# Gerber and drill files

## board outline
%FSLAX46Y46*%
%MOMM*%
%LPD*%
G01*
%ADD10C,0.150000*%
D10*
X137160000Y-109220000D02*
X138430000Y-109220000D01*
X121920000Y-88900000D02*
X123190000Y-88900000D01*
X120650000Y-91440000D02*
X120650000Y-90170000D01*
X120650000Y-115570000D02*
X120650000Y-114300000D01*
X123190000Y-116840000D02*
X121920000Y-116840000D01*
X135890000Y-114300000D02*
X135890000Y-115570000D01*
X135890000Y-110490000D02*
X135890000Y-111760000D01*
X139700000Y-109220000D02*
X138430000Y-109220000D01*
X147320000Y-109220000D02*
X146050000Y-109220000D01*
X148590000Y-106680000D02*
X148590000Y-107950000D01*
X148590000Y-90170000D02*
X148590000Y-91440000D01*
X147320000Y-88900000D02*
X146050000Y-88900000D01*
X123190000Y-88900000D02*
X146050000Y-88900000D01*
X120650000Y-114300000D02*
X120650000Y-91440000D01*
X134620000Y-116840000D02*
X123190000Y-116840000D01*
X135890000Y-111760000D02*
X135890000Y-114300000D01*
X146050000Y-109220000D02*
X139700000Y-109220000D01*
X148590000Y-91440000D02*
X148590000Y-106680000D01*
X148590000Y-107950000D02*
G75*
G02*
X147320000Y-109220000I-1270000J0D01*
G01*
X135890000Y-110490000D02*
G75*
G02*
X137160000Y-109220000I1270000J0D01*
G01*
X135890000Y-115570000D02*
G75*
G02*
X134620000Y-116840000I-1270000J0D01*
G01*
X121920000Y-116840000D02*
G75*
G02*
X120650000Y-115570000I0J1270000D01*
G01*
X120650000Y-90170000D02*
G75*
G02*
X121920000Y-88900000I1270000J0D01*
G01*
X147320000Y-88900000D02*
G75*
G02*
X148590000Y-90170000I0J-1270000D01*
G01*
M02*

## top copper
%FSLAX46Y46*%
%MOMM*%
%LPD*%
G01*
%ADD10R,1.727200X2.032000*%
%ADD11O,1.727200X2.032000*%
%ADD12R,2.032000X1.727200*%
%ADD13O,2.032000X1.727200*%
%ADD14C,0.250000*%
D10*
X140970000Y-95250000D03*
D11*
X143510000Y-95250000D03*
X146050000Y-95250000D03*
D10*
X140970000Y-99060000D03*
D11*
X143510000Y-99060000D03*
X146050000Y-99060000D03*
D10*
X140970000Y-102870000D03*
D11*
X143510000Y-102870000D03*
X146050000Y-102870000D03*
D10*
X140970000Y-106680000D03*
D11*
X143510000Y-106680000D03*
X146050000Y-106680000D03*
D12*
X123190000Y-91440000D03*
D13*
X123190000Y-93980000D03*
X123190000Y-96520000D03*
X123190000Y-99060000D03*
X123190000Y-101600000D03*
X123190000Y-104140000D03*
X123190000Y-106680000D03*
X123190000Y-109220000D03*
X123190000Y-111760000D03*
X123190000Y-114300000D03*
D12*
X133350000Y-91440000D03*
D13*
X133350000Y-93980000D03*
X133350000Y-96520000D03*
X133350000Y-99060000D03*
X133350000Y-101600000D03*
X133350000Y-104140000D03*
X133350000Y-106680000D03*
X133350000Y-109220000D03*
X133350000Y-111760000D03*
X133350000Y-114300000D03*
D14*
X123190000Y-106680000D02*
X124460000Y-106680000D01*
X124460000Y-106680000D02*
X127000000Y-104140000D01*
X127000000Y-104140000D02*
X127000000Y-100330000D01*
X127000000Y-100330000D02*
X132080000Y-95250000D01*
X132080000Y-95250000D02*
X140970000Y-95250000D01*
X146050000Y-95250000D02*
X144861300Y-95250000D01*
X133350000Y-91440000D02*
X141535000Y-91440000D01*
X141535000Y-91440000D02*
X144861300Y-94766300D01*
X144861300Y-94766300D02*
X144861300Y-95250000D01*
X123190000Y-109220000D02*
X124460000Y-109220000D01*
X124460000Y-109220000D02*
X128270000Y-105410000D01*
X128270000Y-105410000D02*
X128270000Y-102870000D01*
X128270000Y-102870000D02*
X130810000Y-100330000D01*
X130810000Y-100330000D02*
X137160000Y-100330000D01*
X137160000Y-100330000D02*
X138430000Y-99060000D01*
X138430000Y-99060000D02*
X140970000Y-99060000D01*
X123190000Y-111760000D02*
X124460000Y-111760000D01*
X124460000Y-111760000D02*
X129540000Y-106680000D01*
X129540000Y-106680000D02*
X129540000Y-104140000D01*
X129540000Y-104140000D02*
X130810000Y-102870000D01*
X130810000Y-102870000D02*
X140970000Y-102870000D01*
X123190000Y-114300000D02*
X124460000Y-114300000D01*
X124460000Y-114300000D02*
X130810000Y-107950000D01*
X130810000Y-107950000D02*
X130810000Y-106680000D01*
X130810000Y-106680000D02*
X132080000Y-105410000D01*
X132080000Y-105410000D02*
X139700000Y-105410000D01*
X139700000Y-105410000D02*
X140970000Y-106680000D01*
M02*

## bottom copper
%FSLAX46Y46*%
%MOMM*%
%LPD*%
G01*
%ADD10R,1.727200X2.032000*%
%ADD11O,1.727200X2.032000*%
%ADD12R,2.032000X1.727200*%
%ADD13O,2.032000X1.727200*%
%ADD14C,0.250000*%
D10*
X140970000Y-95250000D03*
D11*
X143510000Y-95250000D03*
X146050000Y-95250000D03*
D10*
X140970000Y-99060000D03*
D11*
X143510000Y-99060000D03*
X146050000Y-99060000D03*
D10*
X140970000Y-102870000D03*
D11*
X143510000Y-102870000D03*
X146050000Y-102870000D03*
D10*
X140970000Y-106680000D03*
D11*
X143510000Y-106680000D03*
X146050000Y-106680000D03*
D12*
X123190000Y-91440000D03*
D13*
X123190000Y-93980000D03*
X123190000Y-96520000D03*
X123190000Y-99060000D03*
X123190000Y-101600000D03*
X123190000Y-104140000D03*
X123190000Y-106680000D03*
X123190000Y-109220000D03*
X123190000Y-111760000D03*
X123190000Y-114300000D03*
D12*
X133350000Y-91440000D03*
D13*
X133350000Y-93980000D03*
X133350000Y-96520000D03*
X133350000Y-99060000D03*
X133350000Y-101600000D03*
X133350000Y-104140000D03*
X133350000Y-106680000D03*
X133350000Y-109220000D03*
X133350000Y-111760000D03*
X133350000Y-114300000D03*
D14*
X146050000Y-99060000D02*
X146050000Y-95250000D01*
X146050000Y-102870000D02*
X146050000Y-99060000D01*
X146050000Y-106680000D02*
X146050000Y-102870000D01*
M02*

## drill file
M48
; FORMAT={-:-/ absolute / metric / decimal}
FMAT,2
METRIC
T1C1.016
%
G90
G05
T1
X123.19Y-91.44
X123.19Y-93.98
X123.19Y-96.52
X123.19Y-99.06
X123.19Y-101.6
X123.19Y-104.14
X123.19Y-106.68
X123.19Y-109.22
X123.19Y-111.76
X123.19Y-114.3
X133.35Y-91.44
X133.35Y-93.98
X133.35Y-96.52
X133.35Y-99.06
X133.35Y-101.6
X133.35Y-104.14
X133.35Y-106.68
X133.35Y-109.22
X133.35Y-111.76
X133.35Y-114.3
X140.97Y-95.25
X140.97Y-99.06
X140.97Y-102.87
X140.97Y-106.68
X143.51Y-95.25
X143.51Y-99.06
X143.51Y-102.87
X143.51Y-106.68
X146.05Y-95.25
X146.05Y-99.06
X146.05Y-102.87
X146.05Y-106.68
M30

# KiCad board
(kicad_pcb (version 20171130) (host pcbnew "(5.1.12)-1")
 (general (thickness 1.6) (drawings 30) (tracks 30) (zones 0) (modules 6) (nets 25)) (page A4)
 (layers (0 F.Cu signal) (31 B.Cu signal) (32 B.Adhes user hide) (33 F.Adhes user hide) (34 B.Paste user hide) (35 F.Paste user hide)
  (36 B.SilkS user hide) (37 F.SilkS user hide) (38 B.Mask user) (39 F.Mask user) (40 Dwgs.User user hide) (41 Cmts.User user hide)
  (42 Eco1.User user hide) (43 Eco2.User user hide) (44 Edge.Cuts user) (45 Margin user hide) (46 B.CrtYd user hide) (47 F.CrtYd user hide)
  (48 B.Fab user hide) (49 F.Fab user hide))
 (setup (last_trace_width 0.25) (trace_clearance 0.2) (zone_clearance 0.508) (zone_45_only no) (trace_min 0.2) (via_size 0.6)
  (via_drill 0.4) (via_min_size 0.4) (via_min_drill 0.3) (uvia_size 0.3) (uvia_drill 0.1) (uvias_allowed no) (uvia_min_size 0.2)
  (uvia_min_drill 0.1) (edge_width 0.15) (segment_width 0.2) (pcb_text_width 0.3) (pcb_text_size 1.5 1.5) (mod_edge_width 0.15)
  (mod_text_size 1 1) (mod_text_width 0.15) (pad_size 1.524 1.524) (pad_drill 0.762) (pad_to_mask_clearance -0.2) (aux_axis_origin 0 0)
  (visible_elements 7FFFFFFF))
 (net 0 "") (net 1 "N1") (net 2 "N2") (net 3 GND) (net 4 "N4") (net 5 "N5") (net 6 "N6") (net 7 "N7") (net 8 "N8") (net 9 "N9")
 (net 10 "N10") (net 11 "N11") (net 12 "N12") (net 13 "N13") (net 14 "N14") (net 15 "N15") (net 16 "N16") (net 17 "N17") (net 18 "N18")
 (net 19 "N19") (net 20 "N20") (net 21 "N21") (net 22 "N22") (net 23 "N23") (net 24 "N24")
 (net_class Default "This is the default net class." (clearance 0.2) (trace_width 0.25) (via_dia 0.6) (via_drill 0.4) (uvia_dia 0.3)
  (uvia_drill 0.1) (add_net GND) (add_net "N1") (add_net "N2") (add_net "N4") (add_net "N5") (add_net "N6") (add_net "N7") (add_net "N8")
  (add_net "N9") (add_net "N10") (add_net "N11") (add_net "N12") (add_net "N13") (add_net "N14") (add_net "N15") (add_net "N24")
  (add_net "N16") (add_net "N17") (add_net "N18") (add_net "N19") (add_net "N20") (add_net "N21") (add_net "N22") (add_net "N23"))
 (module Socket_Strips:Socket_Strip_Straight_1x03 (layer F.Cu) (at 140.97 95.25)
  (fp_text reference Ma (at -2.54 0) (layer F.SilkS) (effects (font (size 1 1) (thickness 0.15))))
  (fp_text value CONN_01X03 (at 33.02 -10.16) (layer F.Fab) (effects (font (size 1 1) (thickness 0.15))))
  (pad 1 thru_hole rect (at 0 0) (size 1.7272 2.032) (drill 1.016) (layers *.Cu *.Mask F.SilkS) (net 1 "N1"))
  (pad 2 thru_hole oval (at 2.54 0) (size 1.7272 2.032) (drill 1.016) (layers *.Cu *.Mask F.SilkS) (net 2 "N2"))
  (pad 3 thru_hole oval (at 5.08 0) (size 1.7272 2.032) (drill 1.016) (layers *.Cu *.Mask F.SilkS) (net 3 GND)))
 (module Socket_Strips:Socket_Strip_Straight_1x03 (layer F.Cu) (at 140.97 99.06)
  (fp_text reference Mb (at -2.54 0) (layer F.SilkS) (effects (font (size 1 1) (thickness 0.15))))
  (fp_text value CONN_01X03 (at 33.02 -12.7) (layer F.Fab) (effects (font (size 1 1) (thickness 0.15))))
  (pad 1 thru_hole rect (at 0 0) (size 1.7272 2.032) (drill 1.016) (layers *.Cu *.Mask F.SilkS) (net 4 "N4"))
  (pad 2 thru_hole oval (at 2.54 0) (size 1.7272 2.032) (drill 1.016) (layers *.Cu *.Mask F.SilkS) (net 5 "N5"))
  (pad 3 thru_hole oval (at 5.08 0) (size 1.7272 2.032) (drill 1.016) (layers *.Cu *.Mask F.SilkS) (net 3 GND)))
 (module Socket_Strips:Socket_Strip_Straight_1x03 (layer F.Cu) (at 140.97 102.87)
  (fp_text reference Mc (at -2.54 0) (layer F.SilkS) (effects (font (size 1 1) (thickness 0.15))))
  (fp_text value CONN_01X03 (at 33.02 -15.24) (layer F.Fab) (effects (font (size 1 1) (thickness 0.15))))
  (pad 1 thru_hole rect (at 0 0) (size 1.7272 2.032) (drill 1.016) (layers *.Cu *.Mask F.SilkS) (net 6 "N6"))
  (pad 2 thru_hole oval (at 2.54 0) (size 1.7272 2.032) (drill 1.016) (layers *.Cu *.Mask F.SilkS) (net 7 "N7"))
  (pad 3 thru_hole oval (at 5.08 0) (size 1.7272 2.032) (drill 1.016) (layers *.Cu *.Mask F.SilkS) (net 3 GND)))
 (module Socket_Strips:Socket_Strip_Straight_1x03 (layer F.Cu) (at 140.97 106.68)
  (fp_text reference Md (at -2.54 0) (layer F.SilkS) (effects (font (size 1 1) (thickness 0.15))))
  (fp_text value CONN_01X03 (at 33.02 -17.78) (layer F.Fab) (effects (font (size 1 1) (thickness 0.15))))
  (pad 1 thru_hole rect (at 0 0) (size 1.7272 2.032) (drill 1.016) (layers *.Cu *.Mask F.SilkS) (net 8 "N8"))
  (pad 2 thru_hole oval (at 2.54 0) (size 1.7272 2.032) (drill 1.016) (layers *.Cu *.Mask F.SilkS) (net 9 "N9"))
  (pad 3 thru_hole oval (at 5.08 0) (size 1.7272 2.032) (drill 1.016) (layers *.Cu *.Mask F.SilkS) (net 3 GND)))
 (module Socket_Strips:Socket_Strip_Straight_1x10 (layer F.Cu) (at 123.19 91.44 270)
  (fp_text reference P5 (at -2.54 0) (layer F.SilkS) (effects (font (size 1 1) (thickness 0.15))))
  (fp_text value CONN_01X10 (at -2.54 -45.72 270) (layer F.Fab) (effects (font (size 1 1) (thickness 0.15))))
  (pad 1 thru_hole rect (at 0 0 270) (size 1.7272 2.032) (drill 1.016) (layers *.Cu *.Mask F.SilkS) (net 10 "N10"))
  (pad 2 thru_hole oval (at 2.54 0 270) (size 1.7272 2.032) (drill 1.016) (layers *.Cu *.Mask F.SilkS) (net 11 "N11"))
  (pad 3 thru_hole oval (at 5.08 0 270) (size 1.7272 2.032) (drill 1.016) (layers *.Cu *.Mask F.SilkS) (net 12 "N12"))
  (pad 4 thru_hole oval (at 7.62 0 270) (size 1.7272 2.032) (drill 1.016) (layers *.Cu *.Mask F.SilkS) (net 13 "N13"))
  (pad 5 thru_hole oval (at 10.16 0 270) (size 1.7272 2.032) (drill 1.016) (layers *.Cu *.Mask F.SilkS) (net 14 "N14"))
  (pad 6 thru_hole oval (at 12.7 0 270) (size 1.7272 2.032) (drill 1.016) (layers *.Cu *.Mask F.SilkS) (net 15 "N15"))
  (pad 7 thru_hole oval (at 15.24 0 270) (size 1.7272 2.032) (drill 1.016) (layers *.Cu *.Mask F.SilkS) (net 1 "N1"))
  (pad 8 thru_hole oval (at 17.78 0 270) (size 1.7272 2.032) (drill 1.016) (layers *.Cu *.Mask F.SilkS) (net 4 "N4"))
  (pad 9 thru_hole oval (at 20.32 0 270) (size 1.7272 2.032) (drill 1.016) (layers *.Cu *.Mask F.SilkS) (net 6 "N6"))
  (pad 10 thru_hole oval (at 22.86 0 270) (size 1.7272 2.032) (drill 1.016) (layers *.Cu *.Mask F.SilkS) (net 8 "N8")))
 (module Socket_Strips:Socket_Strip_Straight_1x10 (layer F.Cu) (at 133.35 91.44 270)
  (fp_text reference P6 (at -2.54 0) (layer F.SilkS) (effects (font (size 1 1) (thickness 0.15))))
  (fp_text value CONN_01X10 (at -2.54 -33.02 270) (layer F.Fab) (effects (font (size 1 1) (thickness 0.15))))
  (pad 1 thru_hole rect (at 0 0 270) (size 1.7272 2.032) (drill 1.016) (layers *.Cu *.Mask F.SilkS) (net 3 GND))
  (pad 2 thru_hole oval (at 2.54 0 270) (size 1.7272 2.032) (drill 1.016) (layers *.Cu *.Mask F.SilkS) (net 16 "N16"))
  (pad 3 thru_hole oval (at 5.08 0 270) (size 1.7272 2.032) (drill 1.016) (layers *.Cu *.Mask F.SilkS) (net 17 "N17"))
  (pad 4 thru_hole oval (at 7.62 0 270) (size 1.7272 2.032) (drill 1.016) (layers *.Cu *.Mask F.SilkS) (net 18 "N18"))
  (pad 5 thru_hole oval (at 10.16 0 270) (size 1.7272 2.032) (drill 1.016) (layers *.Cu *.Mask F.SilkS) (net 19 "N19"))
  (pad 6 thru_hole oval (at 12.7 0 270) (size 1.7272 2.032) (drill 1.016) (layers *.Cu *.Mask F.SilkS) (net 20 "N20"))
  (pad 7 thru_hole oval (at 15.24 0 270) (size 1.7272 2.032) (drill 1.016) (layers *.Cu *.Mask F.SilkS) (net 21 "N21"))
  (pad 8 thru_hole oval (at 17.78 0 270) (size 1.7272 2.032) (drill 1.016) (layers *.Cu *.Mask F.SilkS) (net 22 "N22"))
  (pad 9 thru_hole oval (at 20.32 0 270) (size 1.7272 2.032) (drill 1.016) (layers *.Cu *.Mask F.SilkS) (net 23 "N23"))
  (pad 10 thru_hole oval (at 22.86 0 270) (size 1.7272 2.032) (drill 1.016) (layers *.Cu *.Mask F.SilkS) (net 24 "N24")))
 (gr_line (start 137.16 109.22) (end 138.43 109.22) (angle 90) (layer Edge.Cuts) (width 0.15))
 (gr_line (start 121.92 88.9) (end 123.19 88.9) (angle 90) (layer Edge.Cuts) (width 0.15))
 (gr_line (start 120.65 91.44) (end 120.65 90.17) (angle 90) (layer Edge.Cuts) (width 0.15))
 (gr_line (start 120.65 115.57) (end 120.65 114.3) (angle 90) (layer Edge.Cuts) (width 0.15))
 (gr_line (start 123.19 116.84) (end 121.92 116.84) (angle 90) (layer Edge.Cuts) (width 0.15))
 (gr_line (start 135.89 114.3) (end 135.89 115.57) (angle 90) (layer Edge.Cuts) (width 0.15))
 (gr_line (start 135.89 110.49) (end 135.89 111.76) (angle 90) (layer Edge.Cuts) (width 0.15))
 (gr_line (start 139.7 109.22) (end 138.43 109.22) (angle 90) (layer Edge.Cuts) (width 0.15))
 (gr_line (start 147.32 109.22) (end 146.05 109.22) (angle 90) (layer Edge.Cuts) (width 0.15))
 (gr_line (start 148.59 106.68) (end 148.59 107.95) (angle 90) (layer Edge.Cuts) (width 0.15))
 (gr_line (start 148.59 90.17) (end 148.59 91.44) (angle 90) (layer Edge.Cuts) (width 0.15))
 (gr_line (start 147.32 88.9) (end 146.05 88.9) (angle 90) (layer Edge.Cuts) (width 0.15))
 (gr_line (start 123.19 88.9) (end 146.05 88.9) (angle 90) (layer Edge.Cuts) (width 0.15))
 (gr_line (start 120.65 114.3) (end 120.65 91.44) (angle 90) (layer Edge.Cuts) (width 0.15))
 (gr_line (start 134.62 116.84) (end 123.19 116.84) (angle 90) (layer Edge.Cuts) (width 0.15))
 (gr_line (start 135.89 111.76) (end 135.89 114.3) (angle 90) (layer Edge.Cuts) (width 0.15))
 (gr_line (start 146.05 109.22) (end 139.7 109.22) (angle 90) (layer Edge.Cuts) (width 0.15))
 (gr_line (start 148.59 91.44) (end 148.59 106.68) (angle 90) (layer Edge.Cuts) (width 0.15))
 (gr_arc (start 147.32 107.95) (end 148.59 107.95) (angle 90) (layer Edge.Cuts) (width 0.15))
 (gr_arc (start 137.16 110.49) (end 135.89 110.49) (angle 90) (layer Edge.Cuts) (width 0.15))
 (gr_arc (start 134.62 115.57) (end 135.89 115.57) (angle 90) (layer Edge.Cuts) (width 0.15))
 (gr_arc (start 121.92 115.57) (end 121.92 116.84) (angle 90) (layer Edge.Cuts) (width 0.15))
 (gr_arc (start 121.92 90.17) (end 120.65 90.17) (angle 90) (layer Edge.Cuts) (width 0.15))
 (gr_arc (start 147.32 90.17) (end 147.32 88.9) (angle 90) (layer Edge.Cuts) (width 0.15))
 (segment (start 123.19 106.68) (end 124.46 106.68) (width 0.25) (layer F.Cu) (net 1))
 (segment (start 124.46 106.68) (end 127 104.14) (width 0.25) (layer F.Cu) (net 1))
 (segment (start 127 104.14) (end 127 100.33) (width 0.25) (layer F.Cu) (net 1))
 (segment (start 127 100.33) (end 132.08 95.25) (width 0.25) (layer F.Cu) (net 1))
 (segment (start 132.08 95.25) (end 140.97 95.25) (width 0.25) (layer F.Cu) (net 1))
 (segment (start 146.05 99.06) (end 146.05 95.25) (width 0.25) (layer B.Cu) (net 3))
 (segment (start 146.05 102.87) (end 146.05 99.06) (width 0.25) (layer B.Cu) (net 3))
 (segment (start 146.05 106.68) (end 146.05 102.87) (width 0.25) (layer B.Cu) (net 3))
 (segment (start 146.05 95.25) (end 144.8613 95.25) (width 0.25) (layer F.Cu) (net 3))
 (segment (start 133.35 91.44) (end 141.535 91.44) (width 0.25) (layer F.Cu) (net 3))
 (segment (start 141.535 91.44) (end 144.8613 94.7663) (width 0.25) (layer F.Cu) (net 3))
 (segment (start 144.8613 94.7663) (end 144.8613 95.25) (width 0.25) (layer F.Cu) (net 3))
 (segment (start 123.19 109.22) (end 124.46 109.22) (width 0.25) (layer F.Cu) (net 4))
 (segment (start 124.46 109.22) (end 128.27 105.41) (width 0.25) (layer F.Cu) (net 4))
 (segment (start 128.27 105.41) (end 128.27 102.87) (width 0.25) (layer F.Cu) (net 4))
 (segment (start 128.27 102.87) (end 130.81 100.33) (width 0.25) (layer F.Cu) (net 4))
 (segment (start 130.81 100.33) (end 137.16 100.33) (width 0.25) (layer F.Cu) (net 4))
 (segment (start 137.16 100.33) (end 138.43 99.06) (width 0.25) (layer F.Cu) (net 4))
 (segment (start 138.43 99.06) (end 140.97 99.06) (width 0.25) (layer F.Cu) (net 4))
 (segment (start 123.19 111.76) (end 124.46 111.76) (width 0.25) (layer F.Cu) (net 6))
 (segment (start 124.46 111.76) (end 129.54 106.68) (width 0.25) (layer F.Cu) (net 6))
 (segment (start 129.54 106.68) (end 129.54 104.14) (width 0.25) (layer F.Cu) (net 6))
 (segment (start 129.54 104.14) (end 130.81 102.87) (width 0.25) (layer F.Cu) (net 6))
 (segment (start 130.81 102.87) (end 140.97 102.87) (width 0.25) (layer F.Cu) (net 6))
 (segment (start 123.19 114.3) (end 124.46 114.3) (width 0.25) (layer F.Cu) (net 8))
 (segment (start 124.46 114.3) (end 130.81 107.95) (width 0.25) (layer F.Cu) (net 8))
 (segment (start 130.81 107.95) (end 130.81 106.68) (width 0.25) (layer F.Cu) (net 8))
 (segment (start 130.81 106.68) (end 132.08 105.41) (width 0.25) (layer F.Cu) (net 8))
 (segment (start 132.08 105.41) (end 139.7 105.41) (width 0.25) (layer F.Cu) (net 8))
 (segment (start 139.7 105.41) (end 140.97 106.68) (width 0.25) (layer F.Cu) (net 8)))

